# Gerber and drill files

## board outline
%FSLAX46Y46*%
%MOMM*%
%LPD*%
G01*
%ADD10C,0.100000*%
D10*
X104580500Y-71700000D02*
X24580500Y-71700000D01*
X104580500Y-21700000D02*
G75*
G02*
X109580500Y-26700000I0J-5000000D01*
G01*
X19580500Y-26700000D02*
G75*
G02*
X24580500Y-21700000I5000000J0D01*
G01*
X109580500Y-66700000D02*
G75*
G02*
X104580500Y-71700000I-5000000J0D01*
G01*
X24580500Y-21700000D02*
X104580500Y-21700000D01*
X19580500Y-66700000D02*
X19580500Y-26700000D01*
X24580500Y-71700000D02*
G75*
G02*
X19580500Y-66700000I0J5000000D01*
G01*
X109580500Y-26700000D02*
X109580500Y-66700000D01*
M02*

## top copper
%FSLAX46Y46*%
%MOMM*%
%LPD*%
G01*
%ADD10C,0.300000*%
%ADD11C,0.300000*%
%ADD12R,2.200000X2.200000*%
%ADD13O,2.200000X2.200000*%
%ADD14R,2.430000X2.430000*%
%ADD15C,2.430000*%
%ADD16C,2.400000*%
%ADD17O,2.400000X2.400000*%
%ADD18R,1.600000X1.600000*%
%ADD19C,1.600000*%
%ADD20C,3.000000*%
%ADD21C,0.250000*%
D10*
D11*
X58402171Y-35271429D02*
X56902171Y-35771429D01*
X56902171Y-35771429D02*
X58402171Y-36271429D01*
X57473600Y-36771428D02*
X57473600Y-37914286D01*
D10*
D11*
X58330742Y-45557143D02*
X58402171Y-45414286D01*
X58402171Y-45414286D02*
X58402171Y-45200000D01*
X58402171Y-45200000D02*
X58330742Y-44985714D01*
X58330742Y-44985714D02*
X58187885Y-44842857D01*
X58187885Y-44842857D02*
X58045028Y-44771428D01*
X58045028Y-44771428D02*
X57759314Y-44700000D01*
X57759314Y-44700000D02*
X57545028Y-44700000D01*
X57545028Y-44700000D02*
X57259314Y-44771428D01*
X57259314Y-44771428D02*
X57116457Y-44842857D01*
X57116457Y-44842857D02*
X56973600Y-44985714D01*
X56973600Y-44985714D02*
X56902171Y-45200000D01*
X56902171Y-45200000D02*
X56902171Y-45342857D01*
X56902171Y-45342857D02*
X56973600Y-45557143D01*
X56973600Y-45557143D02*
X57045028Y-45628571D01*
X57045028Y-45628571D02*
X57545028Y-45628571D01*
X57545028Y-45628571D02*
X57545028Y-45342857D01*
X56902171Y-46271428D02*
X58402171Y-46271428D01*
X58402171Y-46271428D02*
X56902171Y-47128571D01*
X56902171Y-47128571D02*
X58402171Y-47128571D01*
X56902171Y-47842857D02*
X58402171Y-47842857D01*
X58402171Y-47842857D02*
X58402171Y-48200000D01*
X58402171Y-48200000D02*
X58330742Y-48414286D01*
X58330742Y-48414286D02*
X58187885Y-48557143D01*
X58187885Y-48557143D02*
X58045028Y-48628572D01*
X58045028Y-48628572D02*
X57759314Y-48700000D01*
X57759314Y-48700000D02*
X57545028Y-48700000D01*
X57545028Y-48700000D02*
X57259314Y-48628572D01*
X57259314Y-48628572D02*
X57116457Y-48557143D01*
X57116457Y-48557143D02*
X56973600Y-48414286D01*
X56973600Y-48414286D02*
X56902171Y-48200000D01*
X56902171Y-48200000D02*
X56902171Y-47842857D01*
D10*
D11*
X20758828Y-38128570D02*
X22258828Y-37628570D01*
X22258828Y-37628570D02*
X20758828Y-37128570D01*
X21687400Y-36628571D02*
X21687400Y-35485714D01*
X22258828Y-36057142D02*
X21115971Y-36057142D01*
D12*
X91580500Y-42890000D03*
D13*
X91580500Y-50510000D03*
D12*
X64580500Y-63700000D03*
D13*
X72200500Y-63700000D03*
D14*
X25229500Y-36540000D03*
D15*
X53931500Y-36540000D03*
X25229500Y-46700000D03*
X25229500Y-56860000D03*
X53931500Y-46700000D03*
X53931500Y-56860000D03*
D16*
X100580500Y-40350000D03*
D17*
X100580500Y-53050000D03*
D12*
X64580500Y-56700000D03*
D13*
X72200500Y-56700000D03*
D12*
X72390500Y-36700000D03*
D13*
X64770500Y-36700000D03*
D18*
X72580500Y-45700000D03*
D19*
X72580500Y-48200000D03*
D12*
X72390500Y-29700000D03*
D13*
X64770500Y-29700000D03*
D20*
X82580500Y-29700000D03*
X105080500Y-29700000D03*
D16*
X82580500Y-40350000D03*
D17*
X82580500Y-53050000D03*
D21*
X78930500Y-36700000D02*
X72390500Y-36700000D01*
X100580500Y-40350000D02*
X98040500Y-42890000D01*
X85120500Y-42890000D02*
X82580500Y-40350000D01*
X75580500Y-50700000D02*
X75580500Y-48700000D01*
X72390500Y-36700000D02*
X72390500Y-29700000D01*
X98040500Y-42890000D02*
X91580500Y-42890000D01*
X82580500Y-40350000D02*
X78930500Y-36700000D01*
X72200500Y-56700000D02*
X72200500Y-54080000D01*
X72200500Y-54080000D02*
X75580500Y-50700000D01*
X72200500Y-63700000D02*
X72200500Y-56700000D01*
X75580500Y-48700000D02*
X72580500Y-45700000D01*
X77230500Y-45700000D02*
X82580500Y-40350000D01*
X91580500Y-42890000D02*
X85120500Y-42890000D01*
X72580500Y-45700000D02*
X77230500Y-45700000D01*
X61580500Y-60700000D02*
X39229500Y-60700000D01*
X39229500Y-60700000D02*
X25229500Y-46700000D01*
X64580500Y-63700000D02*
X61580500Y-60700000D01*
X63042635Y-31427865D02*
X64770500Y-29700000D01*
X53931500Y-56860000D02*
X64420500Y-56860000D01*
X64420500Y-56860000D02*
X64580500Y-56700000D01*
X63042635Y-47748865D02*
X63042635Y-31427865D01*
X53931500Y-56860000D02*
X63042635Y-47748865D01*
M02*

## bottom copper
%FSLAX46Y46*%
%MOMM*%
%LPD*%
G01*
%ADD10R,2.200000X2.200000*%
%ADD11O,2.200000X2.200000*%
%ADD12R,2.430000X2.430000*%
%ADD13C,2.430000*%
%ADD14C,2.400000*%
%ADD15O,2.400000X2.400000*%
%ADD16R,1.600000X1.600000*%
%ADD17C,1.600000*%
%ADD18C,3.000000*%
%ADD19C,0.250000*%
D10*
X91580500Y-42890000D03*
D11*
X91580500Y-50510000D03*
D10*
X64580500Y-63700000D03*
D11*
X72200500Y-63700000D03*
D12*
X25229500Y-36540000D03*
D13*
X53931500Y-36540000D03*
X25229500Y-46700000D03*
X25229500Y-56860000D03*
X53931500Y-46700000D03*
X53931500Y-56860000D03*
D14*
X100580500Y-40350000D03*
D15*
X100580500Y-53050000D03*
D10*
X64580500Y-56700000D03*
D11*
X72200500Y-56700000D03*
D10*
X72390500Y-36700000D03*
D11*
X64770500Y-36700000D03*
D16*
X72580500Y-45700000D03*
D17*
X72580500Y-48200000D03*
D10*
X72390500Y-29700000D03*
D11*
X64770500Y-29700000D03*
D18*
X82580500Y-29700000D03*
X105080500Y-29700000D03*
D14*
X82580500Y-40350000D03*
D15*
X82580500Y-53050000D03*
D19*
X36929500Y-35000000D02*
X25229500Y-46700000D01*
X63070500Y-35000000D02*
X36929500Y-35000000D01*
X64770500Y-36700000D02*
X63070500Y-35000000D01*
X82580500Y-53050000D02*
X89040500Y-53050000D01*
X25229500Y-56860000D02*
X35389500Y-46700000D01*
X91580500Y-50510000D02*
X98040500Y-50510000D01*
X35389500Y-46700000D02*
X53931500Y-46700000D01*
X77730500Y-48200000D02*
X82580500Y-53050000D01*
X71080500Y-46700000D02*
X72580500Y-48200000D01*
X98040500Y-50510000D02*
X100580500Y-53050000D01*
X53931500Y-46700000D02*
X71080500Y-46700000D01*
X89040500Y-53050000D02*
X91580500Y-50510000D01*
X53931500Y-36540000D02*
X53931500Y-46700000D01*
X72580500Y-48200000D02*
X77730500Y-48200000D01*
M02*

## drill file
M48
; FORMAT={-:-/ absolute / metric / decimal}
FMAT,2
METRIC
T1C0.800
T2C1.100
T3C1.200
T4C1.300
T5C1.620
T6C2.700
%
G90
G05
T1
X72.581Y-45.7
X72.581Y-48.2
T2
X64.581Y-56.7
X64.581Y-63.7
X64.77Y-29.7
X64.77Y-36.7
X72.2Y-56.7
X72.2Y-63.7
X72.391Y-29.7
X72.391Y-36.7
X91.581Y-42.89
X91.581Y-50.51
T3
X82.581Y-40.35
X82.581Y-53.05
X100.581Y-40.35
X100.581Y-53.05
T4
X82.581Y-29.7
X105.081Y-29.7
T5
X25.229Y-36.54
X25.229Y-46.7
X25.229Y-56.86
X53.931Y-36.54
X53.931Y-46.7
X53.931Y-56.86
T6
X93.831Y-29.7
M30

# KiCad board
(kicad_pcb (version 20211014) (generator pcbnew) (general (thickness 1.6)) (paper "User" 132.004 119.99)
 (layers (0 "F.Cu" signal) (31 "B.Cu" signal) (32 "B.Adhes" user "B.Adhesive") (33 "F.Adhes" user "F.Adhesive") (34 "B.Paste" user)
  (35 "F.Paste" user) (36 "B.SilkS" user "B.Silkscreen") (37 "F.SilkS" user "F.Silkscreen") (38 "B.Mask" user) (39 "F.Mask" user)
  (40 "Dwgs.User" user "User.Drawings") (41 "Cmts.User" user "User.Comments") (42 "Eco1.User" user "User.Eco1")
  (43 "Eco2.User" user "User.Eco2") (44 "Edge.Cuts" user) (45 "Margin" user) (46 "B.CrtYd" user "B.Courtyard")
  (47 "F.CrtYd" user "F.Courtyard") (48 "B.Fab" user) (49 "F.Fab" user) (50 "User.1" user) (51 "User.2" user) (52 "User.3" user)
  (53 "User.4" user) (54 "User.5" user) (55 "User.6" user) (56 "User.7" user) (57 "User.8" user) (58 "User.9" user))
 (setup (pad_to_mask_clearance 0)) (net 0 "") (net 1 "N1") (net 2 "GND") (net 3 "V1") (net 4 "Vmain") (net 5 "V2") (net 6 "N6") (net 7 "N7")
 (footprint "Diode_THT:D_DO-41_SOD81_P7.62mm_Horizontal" (layer "F.Cu") (at 91.5805 42.89 -90)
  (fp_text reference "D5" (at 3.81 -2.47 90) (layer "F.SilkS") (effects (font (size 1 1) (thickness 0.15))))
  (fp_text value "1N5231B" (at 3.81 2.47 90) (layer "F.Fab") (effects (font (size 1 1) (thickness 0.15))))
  (pad "1" thru_hole rect (at 0 0 270) (size 2.2 2.2) (drill 1.1) (layers *.Cu *.Mask) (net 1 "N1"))
  (pad "2" thru_hole oval (at 7.62 0 270) (size 2.2 2.2) (drill 1.1) (layers *.Cu *.Mask) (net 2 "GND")))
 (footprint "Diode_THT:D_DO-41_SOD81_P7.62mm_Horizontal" (layer "F.Cu") (at 64.5805 63.7)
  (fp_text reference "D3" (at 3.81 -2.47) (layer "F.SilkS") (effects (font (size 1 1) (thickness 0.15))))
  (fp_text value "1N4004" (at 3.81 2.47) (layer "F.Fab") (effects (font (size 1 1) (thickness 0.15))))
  (pad "1" thru_hole rect (at 0 0) (size 2.2 2.2) (drill 1.1) (layers *.Cu *.Mask) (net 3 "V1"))
  (pad "2" thru_hole oval (at 7.62 0) (size 2.2 2.2) (drill 1.1) (layers *.Cu *.Mask) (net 1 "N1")))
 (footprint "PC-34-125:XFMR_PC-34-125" (layer "F.Cu") (at 39.5805 46.7)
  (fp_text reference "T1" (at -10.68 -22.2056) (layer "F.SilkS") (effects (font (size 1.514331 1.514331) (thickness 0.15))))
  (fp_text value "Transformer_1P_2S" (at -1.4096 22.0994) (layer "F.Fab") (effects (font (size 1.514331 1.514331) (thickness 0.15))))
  (pad "1" thru_hole rect locked (at -14.351 -10.16) (size 2.43 2.43) (drill 1.62) (layers *.Cu *.Mask) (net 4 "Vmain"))
  (pad "2" thru_hole circle locked (at 14.351 -10.16) (size 2.43 2.43) (drill 1.62) (layers *.Cu *.Mask) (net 2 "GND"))
  (pad "3" thru_hole circle locked (at -14.351 0) (size 2.43 2.43) (drill 1.62) (layers *.Cu *.Mask) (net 3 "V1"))
  (pad "4" thru_hole circle locked (at -14.351 10.16) (size 2.43 2.43) (drill 1.62) (layers *.Cu *.Mask) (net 2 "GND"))
  (pad "5" thru_hole circle locked (at 14.351 0) (size 2.43 2.43) (drill 1.62) (layers *.Cu *.Mask) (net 2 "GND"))
  (pad "6" thru_hole circle locked (at 14.351 10.16) (size 2.43 2.43) (drill 1.62) (layers *.Cu *.Mask) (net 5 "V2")))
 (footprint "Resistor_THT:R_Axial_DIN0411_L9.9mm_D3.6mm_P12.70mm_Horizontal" (layer "F.Cu") (at 100.5805 40.35 -90)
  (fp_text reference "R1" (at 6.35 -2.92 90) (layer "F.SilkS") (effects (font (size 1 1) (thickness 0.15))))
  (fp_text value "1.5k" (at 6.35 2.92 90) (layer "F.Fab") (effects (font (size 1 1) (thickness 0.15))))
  (pad "1" thru_hole circle (at 0 0 270) (size 2.4 2.4) (drill 1.2) (layers *.Cu *.Mask) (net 1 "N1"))
  (pad "2" thru_hole oval (at 12.7 0 270) (size 2.4 2.4) (drill 1.2) (layers *.Cu *.Mask) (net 2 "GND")))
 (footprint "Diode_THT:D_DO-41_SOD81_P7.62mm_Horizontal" (layer "F.Cu") (at 64.5805 56.7)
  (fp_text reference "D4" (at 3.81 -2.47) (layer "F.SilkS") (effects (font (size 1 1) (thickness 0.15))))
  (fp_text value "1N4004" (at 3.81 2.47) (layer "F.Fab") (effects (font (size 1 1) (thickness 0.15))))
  (pad "1" thru_hole rect (at 0 0) (size 2.2 2.2) (drill 1.1) (layers *.Cu *.Mask) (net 5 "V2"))
  (pad "2" thru_hole oval (at 7.62 0) (size 2.2 2.2) (drill 1.1) (layers *.Cu *.Mask) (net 1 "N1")))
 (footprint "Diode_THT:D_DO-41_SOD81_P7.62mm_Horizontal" (layer "F.Cu") (at 72.3905 36.7 180)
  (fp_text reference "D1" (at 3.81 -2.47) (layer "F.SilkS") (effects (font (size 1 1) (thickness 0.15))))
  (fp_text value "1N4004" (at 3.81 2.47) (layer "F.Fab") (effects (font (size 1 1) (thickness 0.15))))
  (pad "1" thru_hole rect (at 0 0 180) (size 2.2 2.2) (drill 1.1) (layers *.Cu *.Mask) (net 1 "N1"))
  (pad "2" thru_hole oval (at 7.62 0 180) (size 2.2 2.2) (drill 1.1) (layers *.Cu *.Mask) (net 3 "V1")))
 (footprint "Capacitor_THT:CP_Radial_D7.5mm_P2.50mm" (layer "F.Cu") (at 72.5805 45.7 -90)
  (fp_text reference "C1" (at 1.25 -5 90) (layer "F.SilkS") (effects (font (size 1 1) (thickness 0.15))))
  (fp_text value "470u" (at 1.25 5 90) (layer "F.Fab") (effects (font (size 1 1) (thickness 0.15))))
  (pad "1" thru_hole rect (at 0 0 270) (size 1.6 1.6) (drill 0.8) (layers *.Cu *.Mask) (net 1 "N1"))
  (pad "2" thru_hole circle (at 2.5 0 270) (size 1.6 1.6) (drill 0.8) (layers *.Cu *.Mask) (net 2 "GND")))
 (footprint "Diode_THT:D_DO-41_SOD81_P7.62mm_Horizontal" (layer "F.Cu") (at 72.3905 29.7 180)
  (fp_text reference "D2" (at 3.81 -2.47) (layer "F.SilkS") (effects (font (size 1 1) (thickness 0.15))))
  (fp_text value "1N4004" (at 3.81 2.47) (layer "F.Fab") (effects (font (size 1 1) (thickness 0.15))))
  (pad "1" thru_hole rect (at 0 0 180) (size 2.2 2.2) (drill 1.1) (layers *.Cu *.Mask) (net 1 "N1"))
  (pad "2" thru_hole oval (at 7.62 0 180) (size 2.2 2.2) (drill 1.1) (layers *.Cu *.Mask) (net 5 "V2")))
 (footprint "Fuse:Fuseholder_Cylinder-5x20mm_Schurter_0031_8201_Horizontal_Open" (layer "F.Cu") (at 82.5805 29.7)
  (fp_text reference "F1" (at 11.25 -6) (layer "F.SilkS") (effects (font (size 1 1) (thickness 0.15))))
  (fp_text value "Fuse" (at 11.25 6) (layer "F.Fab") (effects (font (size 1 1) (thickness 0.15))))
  (pad "" np_thru_hole circle (at 11.25 0) (size 2.7 2.7) (drill 2.7) (layers *.Cu *.Mask))
  (pad "1" thru_hole circle (at 0 0) (size 3 3) (drill 1.3) (layers *.Cu *.Mask) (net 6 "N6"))
  (pad "2" thru_hole circle (at 22.5 0) (size 3 3) (drill 1.3) (layers *.Cu *.Mask) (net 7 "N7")))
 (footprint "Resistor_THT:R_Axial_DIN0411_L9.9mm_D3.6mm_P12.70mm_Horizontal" (layer "F.Cu") (at 82.5805 40.35 -90)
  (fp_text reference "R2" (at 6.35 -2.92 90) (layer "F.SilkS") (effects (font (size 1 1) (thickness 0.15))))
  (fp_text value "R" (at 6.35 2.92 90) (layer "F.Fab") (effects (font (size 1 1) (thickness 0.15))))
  (pad "1" thru_hole circle (at 0 0 270) (size 2.4 2.4) (drill 1.2) (layers *.Cu *.Mask) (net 1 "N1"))
  (pad "2" thru_hole oval (at 12.7 0 270) (size 2.4 2.4) (drill 1.2) (layers *.Cu *.Mask) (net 2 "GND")))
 (gr_line (start 104.5805 71.7) (end 24.5805 71.7) (layer "Edge.Cuts") (width 0.1))
 (gr_arc (start 104.5805 21.7) (mid 108.116034 23.164466) (end 109.5805 26.7) (layer "Edge.Cuts") (width 0.1))
 (gr_arc (start 19.5805 26.7) (mid 21.044966 23.164466) (end 24.5805 21.7) (layer "Edge.Cuts") (width 0.1))
 (gr_arc (start 109.5805 66.7) (mid 108.116034 70.235534) (end 104.5805 71.7) (layer "Edge.Cuts") (width 0.1))
 (gr_line (start 24.5805 21.7) (end 104.5805 21.7) (layer "Edge.Cuts") (width 0.1))
 (gr_line (start 19.5805 66.7) (end 19.5805 26.7) (layer "Edge.Cuts") (width 0.1))
 (gr_arc (start 24.5805 71.7) (mid 21.044966 70.235534) (end 19.5805 66.7) (layer "Edge.Cuts") (width 0.1))
 (gr_line (start 109.5805 26.7) (end 109.5805 66.7) (layer "Edge.Cuts") (width 0.1))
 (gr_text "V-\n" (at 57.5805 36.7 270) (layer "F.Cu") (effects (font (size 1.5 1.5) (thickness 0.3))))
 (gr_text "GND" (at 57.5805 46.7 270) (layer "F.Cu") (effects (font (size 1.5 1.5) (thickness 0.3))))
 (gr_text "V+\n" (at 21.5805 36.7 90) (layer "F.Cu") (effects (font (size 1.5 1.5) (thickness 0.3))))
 (segment (start 78.9305 36.7) (end 72.3905 36.7) (width 0.25) (layer "F.Cu") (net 1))
 (segment (start 100.5805 40.35) (end 98.0405 42.89) (width 0.25) (layer "F.Cu") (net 1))
 (segment (start 85.1205 42.89) (end 82.5805 40.35) (width 0.25) (layer "F.Cu") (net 1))
 (segment (start 75.5805 50.7) (end 75.5805 48.7) (width 0.25) (layer "F.Cu") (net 1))
 (segment (start 72.3905 36.7) (end 72.3905 29.7) (width 0.25) (layer "F.Cu") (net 1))
 (segment (start 98.0405 42.89) (end 91.5805 42.89) (width 0.25) (layer "F.Cu") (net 1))
 (segment (start 82.5805 40.35) (end 78.9305 36.7) (width 0.25) (layer "F.Cu") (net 1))
 (segment (start 72.2005 56.7) (end 72.2005 54.08) (width 0.25) (layer "F.Cu") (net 1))
 (segment (start 72.2005 54.08) (end 75.5805 50.7) (width 0.25) (layer "F.Cu") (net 1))
 (segment (start 72.2005 63.7) (end 72.2005 56.7) (width 0.25) (layer "F.Cu") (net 1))
 (segment (start 75.5805 48.7) (end 72.5805 45.7) (width 0.25) (layer "F.Cu") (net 1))
 (segment (start 77.2305 45.7) (end 82.5805 40.35) (width 0.25) (layer "F.Cu") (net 1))
 (segment (start 91.5805 42.89) (end 85.1205 42.89) (width 0.25) (layer "F.Cu") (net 1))
 (segment (start 72.5805 45.7) (end 77.2305 45.7) (width 0.25) (layer "F.Cu") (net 1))
 (segment (start 61.5805 60.7) (end 39.2295 60.7) (width 0.25) (layer "F.Cu") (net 3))
 (segment (start 39.2295 60.7) (end 25.2295 46.7) (width 0.25) (layer "F.Cu") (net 3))
 (segment (start 64.5805 63.7) (end 61.5805 60.7) (width 0.25) (layer "F.Cu") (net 3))
 (segment (start 36.9295 35) (end 25.2295 46.7) (width 0.25) (layer "B.Cu") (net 3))
 (segment (start 63.0705 35) (end 36.9295 35) (width 0.25) (layer "B.Cu") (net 3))
 (segment (start 64.7705 36.7) (end 63.0705 35) (width 0.25) (layer "B.Cu") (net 3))
 (segment (start 63.042635 31.427865) (end 64.7705 29.7) (width 0.25) (layer "F.Cu") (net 5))
 (segment (start 53.9315 56.86) (end 64.4205 56.86) (width 0.25) (layer "F.Cu") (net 5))
 (segment (start 64.4205 56.86) (end 64.5805 56.7) (width 0.25) (layer "F.Cu") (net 5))
 (segment (start 63.042635 47.748865) (end 63.042635 31.427865) (width 0.25) (layer "F.Cu") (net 5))
 (segment (start 53.9315 56.86) (end 63.042635 47.748865) (width 0.25) (layer "F.Cu") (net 5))
 (segment (start 82.5805 53.05) (end 89.0405 53.05) (width 0.25) (layer "B.Cu") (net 2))
 (segment (start 25.2295 56.86) (end 35.3895 46.7) (width 0.25) (layer "B.Cu") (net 2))
 (segment (start 91.5805 50.51) (end 98.0405 50.51) (width 0.25) (layer "B.Cu") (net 2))
 (segment (start 35.3895 46.7) (end 53.9315 46.7) (width 0.25) (layer "B.Cu") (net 2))
 (segment (start 77.7305 48.2) (end 82.5805 53.05) (width 0.25) (layer "B.Cu") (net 2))
 (segment (start 71.0805 46.7) (end 72.5805 48.2) (width 0.25) (layer "B.Cu") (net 2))
 (segment (start 98.0405 50.51) (end 100.5805 53.05) (width 0.25) (layer "B.Cu") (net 2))
 (segment (start 53.9315 46.7) (end 71.0805 46.7) (width 0.25) (layer "B.Cu") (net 2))
 (segment (start 89.0405 53.05) (end 91.5805 50.51) (width 0.25) (layer "B.Cu") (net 2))
 (segment (start 53.9315 36.54) (end 53.9315 46.7) (width 0.25) (layer "B.Cu") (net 2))
 (segment (start 72.5805 48.2) (end 77.7305 48.2) (width 0.25) (layer "B.Cu") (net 2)))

